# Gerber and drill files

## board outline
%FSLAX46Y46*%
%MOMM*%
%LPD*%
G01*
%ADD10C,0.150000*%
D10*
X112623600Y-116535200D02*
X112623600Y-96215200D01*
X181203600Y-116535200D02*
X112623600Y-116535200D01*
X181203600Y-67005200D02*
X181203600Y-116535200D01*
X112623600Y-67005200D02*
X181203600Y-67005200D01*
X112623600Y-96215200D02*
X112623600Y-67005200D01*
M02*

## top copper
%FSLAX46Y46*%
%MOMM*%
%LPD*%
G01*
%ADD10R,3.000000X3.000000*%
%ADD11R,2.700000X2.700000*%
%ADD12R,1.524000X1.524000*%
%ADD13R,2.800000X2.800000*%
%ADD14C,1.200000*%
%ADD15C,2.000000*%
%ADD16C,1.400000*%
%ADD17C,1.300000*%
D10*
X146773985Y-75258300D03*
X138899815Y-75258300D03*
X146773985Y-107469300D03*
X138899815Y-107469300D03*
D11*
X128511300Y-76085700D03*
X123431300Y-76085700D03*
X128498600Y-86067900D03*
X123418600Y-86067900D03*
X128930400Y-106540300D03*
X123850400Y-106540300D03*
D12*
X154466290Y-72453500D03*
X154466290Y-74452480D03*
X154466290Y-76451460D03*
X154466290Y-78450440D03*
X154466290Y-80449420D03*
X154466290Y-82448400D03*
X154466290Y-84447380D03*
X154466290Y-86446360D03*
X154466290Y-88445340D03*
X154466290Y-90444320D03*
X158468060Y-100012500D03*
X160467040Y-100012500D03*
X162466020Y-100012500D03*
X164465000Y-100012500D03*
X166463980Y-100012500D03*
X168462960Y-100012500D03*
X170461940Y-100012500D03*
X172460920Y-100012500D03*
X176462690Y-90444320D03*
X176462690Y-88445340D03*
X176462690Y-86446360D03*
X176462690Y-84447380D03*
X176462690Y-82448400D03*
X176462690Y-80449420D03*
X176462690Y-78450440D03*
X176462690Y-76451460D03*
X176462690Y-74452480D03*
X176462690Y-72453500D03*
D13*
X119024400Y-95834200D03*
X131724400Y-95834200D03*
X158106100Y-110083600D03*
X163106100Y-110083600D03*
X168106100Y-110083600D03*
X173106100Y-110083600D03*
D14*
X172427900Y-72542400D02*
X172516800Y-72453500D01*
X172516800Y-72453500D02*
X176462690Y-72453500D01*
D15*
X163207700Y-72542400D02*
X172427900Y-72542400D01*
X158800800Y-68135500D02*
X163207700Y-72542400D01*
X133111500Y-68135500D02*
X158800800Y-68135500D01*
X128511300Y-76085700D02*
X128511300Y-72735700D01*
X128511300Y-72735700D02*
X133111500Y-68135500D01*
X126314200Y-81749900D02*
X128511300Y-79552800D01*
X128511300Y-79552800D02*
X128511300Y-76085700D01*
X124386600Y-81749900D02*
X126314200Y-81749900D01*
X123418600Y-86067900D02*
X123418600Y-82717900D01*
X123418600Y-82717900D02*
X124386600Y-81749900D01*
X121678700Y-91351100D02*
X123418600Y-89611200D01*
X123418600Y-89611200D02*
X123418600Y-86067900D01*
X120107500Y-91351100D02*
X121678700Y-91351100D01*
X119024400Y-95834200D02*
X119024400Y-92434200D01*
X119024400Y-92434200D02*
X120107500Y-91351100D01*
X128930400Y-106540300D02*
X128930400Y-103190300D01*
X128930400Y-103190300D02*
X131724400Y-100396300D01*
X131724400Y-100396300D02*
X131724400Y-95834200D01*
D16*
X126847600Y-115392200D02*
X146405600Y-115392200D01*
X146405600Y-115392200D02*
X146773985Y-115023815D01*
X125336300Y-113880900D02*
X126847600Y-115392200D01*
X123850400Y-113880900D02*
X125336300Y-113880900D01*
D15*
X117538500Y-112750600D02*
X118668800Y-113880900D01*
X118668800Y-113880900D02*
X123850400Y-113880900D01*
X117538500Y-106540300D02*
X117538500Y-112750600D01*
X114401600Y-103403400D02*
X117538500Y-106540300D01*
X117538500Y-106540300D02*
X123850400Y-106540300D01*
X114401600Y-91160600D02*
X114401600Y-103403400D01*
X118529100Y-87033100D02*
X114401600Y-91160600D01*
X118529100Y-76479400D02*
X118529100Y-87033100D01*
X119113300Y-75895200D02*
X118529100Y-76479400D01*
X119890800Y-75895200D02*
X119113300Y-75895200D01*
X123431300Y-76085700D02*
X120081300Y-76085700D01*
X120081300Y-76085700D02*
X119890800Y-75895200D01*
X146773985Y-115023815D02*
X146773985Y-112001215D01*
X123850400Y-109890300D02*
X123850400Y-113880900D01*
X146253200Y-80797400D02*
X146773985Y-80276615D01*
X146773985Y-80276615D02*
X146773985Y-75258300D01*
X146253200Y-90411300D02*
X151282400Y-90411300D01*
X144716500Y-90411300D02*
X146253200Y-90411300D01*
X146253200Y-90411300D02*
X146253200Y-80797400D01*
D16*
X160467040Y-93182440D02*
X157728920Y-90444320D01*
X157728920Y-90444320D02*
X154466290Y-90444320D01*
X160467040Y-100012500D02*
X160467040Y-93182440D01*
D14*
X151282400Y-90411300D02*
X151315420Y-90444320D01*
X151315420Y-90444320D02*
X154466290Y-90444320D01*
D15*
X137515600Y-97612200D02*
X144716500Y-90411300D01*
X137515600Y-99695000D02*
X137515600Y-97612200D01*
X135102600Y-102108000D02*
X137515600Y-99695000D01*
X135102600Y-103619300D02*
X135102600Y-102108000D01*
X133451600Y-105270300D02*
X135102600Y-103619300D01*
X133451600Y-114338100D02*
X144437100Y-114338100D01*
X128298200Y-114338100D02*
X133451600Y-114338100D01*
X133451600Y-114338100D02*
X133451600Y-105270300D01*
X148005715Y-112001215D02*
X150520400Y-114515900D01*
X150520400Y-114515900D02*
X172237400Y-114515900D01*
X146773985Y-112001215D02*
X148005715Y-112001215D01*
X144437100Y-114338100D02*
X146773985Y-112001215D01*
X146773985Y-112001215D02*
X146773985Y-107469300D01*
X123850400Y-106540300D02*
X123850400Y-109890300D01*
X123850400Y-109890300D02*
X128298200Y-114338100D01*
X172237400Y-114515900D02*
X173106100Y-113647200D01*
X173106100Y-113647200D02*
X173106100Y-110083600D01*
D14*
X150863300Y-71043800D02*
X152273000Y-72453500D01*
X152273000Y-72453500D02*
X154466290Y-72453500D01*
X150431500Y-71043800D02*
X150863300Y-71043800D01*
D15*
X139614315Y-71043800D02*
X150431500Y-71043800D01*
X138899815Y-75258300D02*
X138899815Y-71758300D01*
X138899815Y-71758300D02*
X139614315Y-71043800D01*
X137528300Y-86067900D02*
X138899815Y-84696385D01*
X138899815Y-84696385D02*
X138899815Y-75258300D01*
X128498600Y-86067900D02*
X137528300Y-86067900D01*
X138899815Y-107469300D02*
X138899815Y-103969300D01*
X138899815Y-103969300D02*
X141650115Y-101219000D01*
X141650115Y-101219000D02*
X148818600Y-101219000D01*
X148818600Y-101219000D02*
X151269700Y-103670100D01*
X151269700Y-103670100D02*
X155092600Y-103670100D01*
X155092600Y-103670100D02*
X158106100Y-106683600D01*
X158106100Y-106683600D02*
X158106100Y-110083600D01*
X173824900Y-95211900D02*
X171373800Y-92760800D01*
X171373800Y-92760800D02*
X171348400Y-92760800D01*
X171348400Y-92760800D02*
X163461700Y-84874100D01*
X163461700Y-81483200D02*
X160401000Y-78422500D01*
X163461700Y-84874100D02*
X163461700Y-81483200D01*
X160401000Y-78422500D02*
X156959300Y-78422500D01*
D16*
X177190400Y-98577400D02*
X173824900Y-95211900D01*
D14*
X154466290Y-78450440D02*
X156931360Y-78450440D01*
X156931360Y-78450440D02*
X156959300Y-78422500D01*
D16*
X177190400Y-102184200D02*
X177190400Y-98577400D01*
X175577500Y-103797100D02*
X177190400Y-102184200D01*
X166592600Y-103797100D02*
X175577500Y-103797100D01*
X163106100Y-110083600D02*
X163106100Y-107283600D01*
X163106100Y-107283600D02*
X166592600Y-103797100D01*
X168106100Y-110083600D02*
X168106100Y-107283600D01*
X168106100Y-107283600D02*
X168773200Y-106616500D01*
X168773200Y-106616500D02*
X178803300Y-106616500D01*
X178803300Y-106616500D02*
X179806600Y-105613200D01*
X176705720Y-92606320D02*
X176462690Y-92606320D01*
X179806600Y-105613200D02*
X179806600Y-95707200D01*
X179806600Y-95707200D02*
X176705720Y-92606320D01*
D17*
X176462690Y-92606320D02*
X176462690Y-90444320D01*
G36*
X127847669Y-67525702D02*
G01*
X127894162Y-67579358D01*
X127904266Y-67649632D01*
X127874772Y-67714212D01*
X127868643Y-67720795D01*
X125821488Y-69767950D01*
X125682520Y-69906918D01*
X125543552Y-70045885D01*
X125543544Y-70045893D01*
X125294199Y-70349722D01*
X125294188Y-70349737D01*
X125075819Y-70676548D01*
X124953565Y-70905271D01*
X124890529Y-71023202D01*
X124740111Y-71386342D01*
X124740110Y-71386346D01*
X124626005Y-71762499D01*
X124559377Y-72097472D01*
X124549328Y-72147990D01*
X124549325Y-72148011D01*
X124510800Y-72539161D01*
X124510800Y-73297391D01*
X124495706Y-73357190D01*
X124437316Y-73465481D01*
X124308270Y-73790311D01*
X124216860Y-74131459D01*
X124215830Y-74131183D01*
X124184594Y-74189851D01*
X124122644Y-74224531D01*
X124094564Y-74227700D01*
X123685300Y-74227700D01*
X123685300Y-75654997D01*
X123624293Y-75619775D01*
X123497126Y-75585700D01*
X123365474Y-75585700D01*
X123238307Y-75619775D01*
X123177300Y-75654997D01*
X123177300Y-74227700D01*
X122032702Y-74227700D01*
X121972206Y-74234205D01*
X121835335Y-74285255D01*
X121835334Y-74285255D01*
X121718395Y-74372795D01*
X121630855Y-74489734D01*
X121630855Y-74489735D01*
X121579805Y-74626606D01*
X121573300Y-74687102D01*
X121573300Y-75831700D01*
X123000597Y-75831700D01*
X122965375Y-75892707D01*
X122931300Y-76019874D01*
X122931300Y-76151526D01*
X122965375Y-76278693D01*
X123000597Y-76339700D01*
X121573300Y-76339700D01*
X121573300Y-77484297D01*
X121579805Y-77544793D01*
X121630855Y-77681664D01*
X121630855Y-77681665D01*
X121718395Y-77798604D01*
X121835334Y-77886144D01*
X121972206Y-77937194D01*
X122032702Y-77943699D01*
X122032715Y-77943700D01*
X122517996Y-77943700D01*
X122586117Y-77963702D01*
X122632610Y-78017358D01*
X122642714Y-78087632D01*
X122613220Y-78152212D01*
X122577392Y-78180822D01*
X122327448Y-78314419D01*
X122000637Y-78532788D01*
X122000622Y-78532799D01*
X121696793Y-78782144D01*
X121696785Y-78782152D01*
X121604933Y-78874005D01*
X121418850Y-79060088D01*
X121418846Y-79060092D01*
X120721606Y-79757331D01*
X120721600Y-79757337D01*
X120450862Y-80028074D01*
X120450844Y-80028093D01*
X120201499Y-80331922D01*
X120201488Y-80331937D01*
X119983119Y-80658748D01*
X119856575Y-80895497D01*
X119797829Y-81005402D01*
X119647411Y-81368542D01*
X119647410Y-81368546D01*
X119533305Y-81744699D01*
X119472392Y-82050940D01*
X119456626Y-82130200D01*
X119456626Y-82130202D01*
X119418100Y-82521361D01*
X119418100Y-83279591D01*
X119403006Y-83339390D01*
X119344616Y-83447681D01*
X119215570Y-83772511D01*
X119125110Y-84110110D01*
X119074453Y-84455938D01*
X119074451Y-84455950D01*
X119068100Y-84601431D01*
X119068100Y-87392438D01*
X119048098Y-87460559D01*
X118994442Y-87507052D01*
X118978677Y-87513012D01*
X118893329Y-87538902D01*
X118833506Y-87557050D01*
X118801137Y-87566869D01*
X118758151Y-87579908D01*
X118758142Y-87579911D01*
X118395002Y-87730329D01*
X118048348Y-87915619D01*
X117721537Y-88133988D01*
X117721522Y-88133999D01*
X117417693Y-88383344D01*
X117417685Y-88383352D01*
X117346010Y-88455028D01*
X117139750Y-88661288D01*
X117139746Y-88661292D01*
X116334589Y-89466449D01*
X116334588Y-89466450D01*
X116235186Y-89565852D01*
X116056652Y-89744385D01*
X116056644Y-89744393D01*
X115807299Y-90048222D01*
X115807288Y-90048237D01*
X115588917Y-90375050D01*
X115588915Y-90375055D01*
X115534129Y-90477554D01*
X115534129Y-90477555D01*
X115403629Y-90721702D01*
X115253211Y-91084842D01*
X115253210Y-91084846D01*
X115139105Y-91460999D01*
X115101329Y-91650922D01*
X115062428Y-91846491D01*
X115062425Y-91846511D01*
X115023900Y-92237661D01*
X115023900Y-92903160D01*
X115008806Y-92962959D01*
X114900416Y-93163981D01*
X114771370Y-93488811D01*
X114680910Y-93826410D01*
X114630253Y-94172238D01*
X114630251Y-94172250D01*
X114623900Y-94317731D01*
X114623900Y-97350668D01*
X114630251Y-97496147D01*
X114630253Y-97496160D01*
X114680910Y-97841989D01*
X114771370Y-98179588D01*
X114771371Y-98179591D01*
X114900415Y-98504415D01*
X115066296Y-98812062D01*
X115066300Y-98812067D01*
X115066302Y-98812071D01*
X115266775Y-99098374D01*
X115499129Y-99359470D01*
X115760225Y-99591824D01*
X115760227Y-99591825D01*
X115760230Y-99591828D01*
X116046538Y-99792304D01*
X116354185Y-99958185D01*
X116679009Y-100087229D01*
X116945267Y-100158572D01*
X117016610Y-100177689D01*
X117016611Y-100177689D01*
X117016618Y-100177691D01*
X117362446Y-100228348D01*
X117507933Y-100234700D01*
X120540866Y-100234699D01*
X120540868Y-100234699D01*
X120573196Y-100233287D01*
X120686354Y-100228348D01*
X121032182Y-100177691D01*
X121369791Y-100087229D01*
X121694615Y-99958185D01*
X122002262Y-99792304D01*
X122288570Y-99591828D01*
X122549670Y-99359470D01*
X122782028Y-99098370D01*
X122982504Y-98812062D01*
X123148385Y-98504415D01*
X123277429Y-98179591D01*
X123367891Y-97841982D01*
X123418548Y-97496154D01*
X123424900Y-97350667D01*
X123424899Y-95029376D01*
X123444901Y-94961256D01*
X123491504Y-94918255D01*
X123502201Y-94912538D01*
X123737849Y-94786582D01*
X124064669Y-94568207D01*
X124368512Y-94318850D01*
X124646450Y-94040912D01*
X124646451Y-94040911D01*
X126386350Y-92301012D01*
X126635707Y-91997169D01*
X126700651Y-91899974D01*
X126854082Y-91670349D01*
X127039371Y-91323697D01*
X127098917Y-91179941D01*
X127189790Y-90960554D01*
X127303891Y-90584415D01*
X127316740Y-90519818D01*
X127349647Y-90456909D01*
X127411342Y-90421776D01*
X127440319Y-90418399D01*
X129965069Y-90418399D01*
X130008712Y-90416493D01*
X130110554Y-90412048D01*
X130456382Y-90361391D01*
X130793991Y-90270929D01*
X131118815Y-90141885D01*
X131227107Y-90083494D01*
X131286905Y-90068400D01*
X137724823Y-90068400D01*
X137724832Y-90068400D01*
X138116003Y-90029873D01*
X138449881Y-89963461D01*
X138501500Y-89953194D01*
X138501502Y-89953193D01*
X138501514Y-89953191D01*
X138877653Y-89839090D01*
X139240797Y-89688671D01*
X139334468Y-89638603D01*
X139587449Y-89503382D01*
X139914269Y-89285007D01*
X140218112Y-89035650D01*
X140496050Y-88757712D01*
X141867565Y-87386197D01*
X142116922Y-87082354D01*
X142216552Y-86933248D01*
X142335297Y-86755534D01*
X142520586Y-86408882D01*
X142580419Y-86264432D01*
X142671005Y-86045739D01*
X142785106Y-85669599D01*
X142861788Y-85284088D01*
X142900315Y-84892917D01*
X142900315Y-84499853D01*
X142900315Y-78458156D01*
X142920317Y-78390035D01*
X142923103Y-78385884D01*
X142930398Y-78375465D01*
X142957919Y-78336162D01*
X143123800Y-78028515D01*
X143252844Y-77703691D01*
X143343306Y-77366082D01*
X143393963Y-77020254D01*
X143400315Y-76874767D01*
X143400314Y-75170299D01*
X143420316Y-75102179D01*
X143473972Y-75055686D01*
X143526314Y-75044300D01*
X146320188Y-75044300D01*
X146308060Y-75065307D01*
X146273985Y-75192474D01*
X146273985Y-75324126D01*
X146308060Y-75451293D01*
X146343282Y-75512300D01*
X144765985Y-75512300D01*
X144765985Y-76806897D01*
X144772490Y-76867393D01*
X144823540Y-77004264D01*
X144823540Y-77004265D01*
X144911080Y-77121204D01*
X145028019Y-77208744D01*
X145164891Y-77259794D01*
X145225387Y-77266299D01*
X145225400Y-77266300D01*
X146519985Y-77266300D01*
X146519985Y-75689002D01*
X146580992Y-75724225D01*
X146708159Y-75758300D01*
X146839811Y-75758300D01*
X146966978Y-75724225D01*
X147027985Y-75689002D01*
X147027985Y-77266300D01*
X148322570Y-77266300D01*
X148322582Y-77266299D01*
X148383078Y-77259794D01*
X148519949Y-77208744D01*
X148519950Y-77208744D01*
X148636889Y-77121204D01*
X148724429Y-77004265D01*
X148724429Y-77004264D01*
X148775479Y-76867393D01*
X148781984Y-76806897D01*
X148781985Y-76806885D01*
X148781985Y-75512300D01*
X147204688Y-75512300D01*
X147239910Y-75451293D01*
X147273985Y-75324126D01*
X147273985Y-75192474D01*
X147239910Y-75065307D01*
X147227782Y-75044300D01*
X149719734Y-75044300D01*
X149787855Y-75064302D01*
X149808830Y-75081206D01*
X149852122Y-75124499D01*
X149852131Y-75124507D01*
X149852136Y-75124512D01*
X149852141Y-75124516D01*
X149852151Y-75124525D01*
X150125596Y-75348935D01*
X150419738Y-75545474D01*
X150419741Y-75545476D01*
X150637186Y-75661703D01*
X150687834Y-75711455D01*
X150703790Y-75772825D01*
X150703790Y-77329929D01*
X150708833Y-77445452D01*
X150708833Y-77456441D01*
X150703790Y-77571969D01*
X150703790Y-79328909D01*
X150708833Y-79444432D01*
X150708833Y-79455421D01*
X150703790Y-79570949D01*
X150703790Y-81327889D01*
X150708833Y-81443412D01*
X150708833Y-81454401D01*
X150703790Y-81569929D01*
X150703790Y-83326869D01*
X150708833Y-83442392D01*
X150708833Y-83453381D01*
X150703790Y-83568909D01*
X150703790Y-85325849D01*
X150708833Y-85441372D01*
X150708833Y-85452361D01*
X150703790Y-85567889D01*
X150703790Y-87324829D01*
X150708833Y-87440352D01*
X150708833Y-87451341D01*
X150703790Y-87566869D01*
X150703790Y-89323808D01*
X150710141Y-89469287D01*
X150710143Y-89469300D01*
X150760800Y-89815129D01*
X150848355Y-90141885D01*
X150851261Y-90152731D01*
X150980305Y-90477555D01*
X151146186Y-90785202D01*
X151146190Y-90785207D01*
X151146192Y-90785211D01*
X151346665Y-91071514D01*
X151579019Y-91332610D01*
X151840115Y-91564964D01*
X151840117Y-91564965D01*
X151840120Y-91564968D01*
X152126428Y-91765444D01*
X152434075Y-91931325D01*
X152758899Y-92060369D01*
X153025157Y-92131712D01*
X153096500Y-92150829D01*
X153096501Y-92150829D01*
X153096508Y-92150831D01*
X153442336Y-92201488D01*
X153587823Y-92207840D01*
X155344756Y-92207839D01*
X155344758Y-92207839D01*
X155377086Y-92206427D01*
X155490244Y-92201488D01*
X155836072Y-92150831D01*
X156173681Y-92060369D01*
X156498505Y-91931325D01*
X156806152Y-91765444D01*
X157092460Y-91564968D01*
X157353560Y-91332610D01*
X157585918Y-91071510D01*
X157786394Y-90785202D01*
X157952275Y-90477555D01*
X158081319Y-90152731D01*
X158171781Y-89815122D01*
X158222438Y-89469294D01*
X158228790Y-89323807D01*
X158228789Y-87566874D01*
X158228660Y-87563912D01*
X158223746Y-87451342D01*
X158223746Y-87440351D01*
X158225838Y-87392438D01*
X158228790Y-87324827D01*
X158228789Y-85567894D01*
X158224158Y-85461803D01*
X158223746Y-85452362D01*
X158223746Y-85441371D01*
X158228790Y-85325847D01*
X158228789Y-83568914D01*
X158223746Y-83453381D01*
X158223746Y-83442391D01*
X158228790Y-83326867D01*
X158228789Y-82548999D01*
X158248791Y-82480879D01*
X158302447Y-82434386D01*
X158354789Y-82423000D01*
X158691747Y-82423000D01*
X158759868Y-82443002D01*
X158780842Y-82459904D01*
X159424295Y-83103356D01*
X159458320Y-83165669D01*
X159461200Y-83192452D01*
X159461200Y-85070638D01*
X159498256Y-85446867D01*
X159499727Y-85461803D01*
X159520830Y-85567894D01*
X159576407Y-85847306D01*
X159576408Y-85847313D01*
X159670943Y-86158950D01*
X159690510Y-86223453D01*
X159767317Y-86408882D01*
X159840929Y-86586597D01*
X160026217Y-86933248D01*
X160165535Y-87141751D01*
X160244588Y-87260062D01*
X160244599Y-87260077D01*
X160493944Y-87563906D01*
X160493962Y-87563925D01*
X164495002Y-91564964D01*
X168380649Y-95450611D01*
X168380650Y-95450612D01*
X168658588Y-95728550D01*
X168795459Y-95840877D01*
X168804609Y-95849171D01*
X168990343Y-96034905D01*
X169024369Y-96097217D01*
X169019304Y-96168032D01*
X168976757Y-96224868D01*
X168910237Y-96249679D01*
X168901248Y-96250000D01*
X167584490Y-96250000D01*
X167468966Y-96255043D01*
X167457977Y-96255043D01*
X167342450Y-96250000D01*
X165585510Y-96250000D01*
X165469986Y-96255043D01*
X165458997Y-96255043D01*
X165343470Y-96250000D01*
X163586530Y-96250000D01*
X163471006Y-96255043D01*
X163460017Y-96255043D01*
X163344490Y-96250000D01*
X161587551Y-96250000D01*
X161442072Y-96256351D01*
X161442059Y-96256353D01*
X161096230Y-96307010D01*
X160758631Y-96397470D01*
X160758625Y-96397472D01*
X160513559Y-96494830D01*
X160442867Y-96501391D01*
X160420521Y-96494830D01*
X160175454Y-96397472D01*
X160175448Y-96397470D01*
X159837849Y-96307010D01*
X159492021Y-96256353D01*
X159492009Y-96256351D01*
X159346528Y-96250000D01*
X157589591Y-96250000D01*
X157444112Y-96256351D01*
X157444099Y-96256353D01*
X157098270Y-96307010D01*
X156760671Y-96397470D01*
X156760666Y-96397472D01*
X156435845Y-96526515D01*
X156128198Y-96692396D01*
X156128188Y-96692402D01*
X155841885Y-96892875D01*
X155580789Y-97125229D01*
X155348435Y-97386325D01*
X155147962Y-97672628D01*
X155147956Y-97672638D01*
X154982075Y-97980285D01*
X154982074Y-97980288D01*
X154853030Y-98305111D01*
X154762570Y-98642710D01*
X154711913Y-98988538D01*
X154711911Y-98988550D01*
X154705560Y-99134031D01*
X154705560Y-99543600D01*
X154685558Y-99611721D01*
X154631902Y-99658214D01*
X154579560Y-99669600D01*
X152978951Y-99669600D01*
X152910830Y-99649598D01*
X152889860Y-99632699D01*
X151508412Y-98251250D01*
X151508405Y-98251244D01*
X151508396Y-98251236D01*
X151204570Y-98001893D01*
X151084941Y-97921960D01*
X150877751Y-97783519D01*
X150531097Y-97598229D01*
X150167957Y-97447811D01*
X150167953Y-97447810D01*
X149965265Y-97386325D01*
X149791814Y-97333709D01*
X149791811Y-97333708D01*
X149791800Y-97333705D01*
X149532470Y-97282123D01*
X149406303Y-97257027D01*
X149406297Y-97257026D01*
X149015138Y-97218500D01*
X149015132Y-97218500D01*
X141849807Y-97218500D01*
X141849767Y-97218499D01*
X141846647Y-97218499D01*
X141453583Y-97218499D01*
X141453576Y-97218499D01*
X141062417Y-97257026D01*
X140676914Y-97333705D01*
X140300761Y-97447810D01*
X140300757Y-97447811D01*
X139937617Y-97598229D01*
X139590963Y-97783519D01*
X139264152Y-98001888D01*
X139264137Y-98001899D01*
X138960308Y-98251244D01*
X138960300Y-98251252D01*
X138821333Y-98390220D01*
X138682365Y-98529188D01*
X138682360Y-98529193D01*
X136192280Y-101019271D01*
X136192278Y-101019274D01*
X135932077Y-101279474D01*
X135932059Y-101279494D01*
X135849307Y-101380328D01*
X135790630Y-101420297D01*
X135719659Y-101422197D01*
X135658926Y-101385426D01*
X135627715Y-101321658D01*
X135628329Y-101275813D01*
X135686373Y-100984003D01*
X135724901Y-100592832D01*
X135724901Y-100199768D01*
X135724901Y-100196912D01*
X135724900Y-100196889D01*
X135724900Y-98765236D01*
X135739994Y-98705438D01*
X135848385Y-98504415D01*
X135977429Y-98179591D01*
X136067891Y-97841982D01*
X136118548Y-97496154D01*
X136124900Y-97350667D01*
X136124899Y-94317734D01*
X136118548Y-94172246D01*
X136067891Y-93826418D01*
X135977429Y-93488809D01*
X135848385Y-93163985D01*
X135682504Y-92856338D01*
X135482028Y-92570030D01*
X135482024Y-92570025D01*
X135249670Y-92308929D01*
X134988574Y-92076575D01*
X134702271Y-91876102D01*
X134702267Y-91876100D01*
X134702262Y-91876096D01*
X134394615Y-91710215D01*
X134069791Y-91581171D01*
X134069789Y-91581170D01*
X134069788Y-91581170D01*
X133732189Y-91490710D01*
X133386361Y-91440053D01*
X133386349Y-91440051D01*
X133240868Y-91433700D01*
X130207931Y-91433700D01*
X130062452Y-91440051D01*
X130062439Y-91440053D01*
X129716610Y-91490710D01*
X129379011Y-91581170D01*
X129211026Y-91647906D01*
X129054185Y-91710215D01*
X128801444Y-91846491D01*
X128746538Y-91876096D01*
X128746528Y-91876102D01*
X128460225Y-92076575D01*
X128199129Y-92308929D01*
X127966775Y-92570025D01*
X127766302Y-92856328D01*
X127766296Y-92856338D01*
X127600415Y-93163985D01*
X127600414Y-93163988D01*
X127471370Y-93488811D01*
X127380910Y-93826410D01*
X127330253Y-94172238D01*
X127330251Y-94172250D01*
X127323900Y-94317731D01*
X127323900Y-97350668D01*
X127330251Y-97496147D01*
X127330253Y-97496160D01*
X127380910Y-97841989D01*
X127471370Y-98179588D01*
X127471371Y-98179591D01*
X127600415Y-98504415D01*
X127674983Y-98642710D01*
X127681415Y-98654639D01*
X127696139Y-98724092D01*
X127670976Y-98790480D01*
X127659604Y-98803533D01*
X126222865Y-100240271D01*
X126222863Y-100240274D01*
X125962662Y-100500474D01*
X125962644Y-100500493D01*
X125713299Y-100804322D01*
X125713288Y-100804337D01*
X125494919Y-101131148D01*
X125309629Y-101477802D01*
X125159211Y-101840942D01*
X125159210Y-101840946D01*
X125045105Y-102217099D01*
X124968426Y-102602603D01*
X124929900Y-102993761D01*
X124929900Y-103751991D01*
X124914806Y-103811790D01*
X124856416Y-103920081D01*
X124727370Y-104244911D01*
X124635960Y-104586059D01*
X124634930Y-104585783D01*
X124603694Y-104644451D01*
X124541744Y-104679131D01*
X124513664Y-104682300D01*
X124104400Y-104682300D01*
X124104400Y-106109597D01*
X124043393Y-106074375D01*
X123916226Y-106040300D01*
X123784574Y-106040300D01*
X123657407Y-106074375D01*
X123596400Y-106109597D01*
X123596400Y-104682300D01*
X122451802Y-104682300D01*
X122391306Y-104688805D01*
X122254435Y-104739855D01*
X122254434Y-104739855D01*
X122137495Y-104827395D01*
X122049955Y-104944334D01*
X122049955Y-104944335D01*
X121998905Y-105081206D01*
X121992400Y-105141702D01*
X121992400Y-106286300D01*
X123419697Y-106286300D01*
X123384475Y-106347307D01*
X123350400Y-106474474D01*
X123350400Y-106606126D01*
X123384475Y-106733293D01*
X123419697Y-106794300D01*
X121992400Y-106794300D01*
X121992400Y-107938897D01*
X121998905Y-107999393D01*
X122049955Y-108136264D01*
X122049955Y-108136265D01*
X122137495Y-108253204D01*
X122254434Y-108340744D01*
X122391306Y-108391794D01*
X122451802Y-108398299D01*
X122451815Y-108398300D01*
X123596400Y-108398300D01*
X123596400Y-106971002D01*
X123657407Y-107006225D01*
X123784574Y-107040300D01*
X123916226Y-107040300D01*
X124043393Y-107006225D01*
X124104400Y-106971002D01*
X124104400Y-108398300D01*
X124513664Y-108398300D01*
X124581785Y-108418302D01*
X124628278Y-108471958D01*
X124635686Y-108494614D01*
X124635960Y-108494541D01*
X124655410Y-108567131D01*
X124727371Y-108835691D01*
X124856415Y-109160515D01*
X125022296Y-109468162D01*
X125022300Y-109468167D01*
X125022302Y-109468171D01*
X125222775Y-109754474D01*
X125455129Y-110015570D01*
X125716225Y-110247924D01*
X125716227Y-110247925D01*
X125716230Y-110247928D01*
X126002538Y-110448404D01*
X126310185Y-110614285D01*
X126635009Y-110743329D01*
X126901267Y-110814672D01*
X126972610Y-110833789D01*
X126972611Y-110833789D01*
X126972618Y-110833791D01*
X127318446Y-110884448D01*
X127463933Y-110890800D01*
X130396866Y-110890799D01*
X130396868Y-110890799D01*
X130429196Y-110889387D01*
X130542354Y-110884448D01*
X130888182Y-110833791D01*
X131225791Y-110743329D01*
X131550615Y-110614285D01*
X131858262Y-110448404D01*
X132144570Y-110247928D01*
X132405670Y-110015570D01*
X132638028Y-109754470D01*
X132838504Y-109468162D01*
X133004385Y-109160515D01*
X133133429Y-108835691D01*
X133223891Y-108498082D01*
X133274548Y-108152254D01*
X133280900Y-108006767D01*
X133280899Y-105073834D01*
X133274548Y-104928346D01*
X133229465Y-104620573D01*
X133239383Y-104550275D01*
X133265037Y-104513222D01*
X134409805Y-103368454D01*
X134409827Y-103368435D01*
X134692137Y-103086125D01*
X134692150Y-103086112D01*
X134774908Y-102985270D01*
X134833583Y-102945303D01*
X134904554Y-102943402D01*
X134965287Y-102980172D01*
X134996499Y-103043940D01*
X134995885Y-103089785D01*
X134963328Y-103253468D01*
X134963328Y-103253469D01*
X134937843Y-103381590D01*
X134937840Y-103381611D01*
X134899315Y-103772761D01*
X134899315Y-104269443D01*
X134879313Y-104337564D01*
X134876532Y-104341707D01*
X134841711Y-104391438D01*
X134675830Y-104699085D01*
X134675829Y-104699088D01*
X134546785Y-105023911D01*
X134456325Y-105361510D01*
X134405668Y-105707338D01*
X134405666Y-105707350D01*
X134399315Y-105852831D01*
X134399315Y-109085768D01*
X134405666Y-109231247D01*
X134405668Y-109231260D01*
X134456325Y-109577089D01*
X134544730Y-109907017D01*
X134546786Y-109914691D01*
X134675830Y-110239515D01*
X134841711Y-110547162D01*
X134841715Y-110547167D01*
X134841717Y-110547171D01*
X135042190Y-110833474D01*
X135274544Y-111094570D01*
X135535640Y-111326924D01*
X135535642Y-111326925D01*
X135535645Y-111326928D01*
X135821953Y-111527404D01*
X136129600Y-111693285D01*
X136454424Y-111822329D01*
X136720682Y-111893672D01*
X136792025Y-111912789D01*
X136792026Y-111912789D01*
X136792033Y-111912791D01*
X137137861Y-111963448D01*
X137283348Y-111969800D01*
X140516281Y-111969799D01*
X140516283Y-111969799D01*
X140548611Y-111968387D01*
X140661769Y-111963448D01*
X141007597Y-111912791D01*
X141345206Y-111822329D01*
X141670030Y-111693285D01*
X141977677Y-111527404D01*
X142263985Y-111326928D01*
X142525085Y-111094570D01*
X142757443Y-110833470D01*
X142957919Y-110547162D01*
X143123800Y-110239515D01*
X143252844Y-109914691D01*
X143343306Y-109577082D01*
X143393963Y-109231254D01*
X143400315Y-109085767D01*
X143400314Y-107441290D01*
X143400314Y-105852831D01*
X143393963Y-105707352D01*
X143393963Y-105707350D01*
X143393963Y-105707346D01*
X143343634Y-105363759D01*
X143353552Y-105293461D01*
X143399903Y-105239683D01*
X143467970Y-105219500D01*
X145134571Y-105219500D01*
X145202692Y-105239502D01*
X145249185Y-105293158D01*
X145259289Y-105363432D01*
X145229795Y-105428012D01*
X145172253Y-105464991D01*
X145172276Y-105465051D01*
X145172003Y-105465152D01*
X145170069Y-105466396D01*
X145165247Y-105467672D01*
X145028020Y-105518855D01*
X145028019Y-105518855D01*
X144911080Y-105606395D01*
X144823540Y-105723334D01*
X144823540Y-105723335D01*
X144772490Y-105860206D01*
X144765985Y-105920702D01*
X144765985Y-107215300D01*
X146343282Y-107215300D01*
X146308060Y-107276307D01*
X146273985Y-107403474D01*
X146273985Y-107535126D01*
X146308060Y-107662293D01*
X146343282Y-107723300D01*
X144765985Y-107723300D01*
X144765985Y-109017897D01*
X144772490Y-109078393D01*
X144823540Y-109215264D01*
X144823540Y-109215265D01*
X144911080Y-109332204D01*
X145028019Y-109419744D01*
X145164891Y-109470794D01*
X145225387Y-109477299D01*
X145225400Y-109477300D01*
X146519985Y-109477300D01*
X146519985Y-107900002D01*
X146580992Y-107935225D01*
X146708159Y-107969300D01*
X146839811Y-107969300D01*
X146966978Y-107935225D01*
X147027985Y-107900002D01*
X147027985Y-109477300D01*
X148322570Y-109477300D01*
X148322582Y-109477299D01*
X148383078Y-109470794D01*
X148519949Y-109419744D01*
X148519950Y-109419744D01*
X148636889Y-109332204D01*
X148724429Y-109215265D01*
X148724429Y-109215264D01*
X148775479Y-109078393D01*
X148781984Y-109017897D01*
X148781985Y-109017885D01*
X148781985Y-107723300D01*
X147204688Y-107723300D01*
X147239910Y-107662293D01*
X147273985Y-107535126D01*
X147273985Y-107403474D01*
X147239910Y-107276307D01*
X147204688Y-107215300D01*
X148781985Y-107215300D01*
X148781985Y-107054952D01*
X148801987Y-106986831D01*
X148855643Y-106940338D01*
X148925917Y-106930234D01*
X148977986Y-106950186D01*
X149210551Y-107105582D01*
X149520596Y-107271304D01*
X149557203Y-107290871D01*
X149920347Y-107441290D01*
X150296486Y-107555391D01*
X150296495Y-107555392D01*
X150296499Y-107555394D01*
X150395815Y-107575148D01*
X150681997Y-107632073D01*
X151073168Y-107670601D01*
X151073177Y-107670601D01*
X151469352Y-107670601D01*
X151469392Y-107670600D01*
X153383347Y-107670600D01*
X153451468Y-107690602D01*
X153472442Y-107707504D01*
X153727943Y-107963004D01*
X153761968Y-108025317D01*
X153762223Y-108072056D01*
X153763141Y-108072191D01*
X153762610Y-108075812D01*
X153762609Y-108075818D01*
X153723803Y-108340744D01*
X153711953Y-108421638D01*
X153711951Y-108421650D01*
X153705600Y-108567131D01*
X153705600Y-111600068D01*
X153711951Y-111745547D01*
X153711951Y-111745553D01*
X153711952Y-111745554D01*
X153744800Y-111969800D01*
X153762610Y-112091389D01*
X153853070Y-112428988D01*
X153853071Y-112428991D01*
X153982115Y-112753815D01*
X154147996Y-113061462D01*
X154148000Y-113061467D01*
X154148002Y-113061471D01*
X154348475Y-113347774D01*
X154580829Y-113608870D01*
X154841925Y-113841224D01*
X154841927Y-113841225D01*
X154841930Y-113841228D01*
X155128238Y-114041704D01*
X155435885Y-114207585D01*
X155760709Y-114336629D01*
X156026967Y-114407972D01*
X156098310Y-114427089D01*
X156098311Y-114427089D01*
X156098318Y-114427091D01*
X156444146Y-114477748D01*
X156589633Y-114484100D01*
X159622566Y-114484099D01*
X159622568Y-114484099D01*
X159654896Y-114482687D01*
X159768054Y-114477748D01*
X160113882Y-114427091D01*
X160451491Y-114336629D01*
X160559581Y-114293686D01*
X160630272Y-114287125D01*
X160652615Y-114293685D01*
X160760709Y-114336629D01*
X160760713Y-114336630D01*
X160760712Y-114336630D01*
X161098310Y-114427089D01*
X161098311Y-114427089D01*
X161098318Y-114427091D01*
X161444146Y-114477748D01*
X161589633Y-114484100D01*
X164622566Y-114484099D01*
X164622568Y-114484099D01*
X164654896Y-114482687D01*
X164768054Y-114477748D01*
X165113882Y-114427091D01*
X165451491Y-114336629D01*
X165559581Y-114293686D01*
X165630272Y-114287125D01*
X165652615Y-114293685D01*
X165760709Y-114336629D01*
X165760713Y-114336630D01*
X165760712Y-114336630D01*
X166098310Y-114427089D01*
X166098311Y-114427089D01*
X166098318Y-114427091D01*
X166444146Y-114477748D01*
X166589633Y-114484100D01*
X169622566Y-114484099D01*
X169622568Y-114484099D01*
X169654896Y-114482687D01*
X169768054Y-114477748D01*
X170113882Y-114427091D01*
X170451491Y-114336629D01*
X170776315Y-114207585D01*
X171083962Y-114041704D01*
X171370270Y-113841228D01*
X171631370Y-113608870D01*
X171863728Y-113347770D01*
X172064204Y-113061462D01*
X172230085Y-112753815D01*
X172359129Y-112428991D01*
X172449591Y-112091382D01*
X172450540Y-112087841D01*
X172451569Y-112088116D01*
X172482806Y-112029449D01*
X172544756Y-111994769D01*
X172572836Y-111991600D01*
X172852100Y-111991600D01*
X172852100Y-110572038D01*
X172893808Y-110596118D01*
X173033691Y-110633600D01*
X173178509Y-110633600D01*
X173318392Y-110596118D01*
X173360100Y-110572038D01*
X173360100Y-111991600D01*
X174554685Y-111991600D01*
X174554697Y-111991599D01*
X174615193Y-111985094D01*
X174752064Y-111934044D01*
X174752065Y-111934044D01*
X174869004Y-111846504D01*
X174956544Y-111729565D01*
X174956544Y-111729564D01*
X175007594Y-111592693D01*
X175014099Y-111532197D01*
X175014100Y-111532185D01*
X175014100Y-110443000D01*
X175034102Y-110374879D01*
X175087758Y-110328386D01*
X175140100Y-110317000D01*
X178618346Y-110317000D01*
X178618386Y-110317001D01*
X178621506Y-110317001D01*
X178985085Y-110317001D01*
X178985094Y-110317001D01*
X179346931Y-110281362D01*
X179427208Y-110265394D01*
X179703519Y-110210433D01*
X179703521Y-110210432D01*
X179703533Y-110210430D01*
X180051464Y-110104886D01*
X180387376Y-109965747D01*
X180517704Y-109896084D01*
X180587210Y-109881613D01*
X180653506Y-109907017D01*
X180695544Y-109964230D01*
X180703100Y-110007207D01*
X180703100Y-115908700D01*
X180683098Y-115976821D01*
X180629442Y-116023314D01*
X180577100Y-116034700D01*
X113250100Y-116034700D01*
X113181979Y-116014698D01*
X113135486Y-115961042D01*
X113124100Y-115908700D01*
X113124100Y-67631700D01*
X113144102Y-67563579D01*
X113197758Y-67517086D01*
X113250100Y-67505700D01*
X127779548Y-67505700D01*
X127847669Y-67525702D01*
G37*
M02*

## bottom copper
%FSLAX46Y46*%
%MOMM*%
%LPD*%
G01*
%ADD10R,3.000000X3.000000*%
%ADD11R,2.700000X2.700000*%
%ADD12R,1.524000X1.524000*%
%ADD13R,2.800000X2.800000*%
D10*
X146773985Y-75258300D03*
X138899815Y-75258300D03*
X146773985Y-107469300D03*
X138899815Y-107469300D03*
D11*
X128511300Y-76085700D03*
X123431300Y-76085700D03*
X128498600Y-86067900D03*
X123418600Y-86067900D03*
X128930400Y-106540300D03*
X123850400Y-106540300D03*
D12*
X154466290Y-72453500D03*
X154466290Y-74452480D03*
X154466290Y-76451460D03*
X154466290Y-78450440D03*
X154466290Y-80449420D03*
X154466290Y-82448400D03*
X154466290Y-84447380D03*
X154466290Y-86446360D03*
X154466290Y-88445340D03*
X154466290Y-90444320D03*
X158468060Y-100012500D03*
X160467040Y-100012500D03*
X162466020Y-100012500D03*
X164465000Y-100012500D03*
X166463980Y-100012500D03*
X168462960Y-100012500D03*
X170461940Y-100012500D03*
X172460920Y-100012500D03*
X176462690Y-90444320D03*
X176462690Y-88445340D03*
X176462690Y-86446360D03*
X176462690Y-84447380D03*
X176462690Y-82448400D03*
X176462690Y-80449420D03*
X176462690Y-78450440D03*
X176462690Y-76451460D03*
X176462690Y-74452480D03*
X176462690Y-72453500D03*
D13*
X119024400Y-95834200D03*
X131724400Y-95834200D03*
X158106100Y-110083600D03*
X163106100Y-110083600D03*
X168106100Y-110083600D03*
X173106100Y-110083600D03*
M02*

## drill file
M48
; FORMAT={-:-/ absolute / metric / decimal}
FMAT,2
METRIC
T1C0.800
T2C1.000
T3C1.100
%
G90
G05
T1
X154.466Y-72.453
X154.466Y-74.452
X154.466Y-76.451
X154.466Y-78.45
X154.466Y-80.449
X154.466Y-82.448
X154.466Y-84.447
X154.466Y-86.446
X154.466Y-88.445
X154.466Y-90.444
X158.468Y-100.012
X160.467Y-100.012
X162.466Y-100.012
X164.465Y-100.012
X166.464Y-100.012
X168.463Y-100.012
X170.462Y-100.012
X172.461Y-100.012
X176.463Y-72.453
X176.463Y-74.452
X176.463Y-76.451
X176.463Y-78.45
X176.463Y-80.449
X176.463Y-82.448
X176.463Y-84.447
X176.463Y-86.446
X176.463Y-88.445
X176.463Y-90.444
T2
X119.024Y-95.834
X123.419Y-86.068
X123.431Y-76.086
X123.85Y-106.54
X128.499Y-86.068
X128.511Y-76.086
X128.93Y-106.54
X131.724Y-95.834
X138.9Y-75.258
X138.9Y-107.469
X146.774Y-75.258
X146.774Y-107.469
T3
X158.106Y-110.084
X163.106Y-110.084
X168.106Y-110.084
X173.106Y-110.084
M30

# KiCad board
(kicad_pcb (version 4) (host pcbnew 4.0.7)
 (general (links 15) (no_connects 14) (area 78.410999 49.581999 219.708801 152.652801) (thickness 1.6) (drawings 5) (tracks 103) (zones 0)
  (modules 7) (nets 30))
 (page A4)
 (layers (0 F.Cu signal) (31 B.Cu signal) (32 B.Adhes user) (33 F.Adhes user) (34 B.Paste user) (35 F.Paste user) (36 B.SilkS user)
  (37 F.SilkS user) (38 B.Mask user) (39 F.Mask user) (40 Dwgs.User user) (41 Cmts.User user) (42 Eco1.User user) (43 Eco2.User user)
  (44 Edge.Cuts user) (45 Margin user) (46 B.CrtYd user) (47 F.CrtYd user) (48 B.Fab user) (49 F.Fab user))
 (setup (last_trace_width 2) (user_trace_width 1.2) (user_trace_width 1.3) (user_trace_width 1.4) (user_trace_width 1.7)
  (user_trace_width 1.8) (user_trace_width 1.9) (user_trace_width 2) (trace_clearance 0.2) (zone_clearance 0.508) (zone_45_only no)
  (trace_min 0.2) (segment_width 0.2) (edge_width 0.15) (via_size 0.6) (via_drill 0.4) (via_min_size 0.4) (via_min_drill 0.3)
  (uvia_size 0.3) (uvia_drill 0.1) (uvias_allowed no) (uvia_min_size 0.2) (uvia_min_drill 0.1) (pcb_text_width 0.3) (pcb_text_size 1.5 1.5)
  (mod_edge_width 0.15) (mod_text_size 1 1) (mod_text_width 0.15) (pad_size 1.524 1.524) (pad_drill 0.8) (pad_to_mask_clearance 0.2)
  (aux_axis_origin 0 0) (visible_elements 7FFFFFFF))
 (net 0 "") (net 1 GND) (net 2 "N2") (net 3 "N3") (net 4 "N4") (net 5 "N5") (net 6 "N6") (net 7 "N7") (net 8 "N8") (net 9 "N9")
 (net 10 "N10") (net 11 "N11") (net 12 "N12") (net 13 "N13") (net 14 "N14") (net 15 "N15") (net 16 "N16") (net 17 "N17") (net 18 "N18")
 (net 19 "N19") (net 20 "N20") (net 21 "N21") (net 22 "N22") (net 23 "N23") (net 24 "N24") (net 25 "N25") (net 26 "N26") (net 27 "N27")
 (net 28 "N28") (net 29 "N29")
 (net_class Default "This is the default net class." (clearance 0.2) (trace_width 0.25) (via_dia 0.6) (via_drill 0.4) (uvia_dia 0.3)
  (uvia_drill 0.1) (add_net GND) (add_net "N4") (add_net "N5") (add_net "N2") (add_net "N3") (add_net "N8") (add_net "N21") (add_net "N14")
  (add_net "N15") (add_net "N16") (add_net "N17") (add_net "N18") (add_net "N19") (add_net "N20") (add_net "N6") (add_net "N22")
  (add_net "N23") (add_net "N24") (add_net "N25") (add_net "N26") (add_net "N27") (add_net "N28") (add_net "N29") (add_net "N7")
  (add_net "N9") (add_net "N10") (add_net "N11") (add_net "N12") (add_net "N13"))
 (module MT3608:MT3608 (layer F.Cu) (at 142.8369 91.3638 270)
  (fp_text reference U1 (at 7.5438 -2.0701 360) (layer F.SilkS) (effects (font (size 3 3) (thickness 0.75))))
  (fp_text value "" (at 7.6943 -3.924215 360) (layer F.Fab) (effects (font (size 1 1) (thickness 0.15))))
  (pad 2 thru_hole rect (at -16.1055 -3.937085 270) (size 3 3) (drill 1) (layers *.Cu *.Mask) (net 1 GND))
  (pad 1 thru_hole rect (at -16.1055 3.937085 270) (size 3 3) (drill 1) (layers *.Cu *.Mask) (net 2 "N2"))
  (pad 4 thru_hole rect (at 16.1055 -3.937085 270) (size 3 3) (drill 1) (layers *.Cu *.Mask) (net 1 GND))
  (pad 3 thru_hole rect (at 16.1055 3.937085 270) (size 3 3) (drill 1) (layers *.Cu *.Mask) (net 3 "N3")))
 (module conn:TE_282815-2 (layer F.Cu) (at 125.9713 76.0857 180)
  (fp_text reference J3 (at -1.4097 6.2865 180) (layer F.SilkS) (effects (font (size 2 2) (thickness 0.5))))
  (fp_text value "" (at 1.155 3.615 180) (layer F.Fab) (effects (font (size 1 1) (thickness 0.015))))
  (pad 1 thru_hole rect (at -2.54 0 180) (size 2.7 2.7) (drill 1) (layers *.Cu *.Mask) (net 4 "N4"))
  (pad 2 thru_hole rect (at 2.54 0 180) (size 2.7 2.7) (drill 1) (layers *.Cu *.Mask) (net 1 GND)))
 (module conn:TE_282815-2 (layer F.Cu) (at 125.9586 86.0679 180)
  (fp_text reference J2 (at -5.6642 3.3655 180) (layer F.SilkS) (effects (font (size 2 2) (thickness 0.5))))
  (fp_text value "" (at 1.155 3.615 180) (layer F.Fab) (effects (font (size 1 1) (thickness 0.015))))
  (pad 1 thru_hole rect (at -2.54 0 180) (size 2.7 2.7) (drill 1) (layers *.Cu *.Mask) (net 2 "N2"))
  (pad 2 thru_hole rect (at 2.54 0 180) (size 2.7 2.7) (drill 1) (layers *.Cu *.Mask) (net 4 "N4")))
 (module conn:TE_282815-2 (layer F.Cu) (at 126.3904 106.5403 180)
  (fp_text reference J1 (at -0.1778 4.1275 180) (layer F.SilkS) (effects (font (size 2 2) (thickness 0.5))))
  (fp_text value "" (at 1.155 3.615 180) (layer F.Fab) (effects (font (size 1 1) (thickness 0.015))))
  (pad 1 thru_hole rect (at -2.54 0 180) (size 2.7 2.7) (drill 1) (layers *.Cu *.Mask) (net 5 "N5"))
  (pad 2 thru_hole rect (at 2.54 0 180) (size 2.7 2.7) (drill 1) (layers *.Cu *.Mask) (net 1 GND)))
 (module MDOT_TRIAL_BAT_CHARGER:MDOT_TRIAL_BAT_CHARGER (layer F.Cu) (at 165.46449 85.44687)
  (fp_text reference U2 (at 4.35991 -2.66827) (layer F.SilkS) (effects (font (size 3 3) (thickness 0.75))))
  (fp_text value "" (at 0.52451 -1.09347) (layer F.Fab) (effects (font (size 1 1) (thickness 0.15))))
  (pad 1 thru_hole rect (at -10.9982 -12.99337) (size 1.524 1.524) (drill 0.8) (layers *.Cu *.Mask) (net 2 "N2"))
  (pad 2 thru_hole rect (at -10.9982 -10.99439) (size 1.524 1.524) (drill 0.8) (layers *.Cu *.Mask) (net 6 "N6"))
  (pad 3 thru_hole rect (at -10.9982 -8.99541) (size 1.524 1.524) (drill 0.8) (layers *.Cu *.Mask) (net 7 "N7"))
  (pad 4 thru_hole rect (at -10.9982 -6.99643) (size 1.524 1.524) (drill 0.8) (layers *.Cu *.Mask) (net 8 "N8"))
  (pad 5 thru_hole rect (at -10.9982 -4.99745) (size 1.524 1.524) (drill 0.8) (layers *.Cu *.Mask) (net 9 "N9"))
  (pad 6 thru_hole rect (at -10.9982 -2.99847) (size 1.524 1.524) (drill 0.8) (layers *.Cu *.Mask) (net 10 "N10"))
  (pad 7 thru_hole rect (at -10.9982 -0.99949) (size 1.524 1.524) (drill 0.8) (layers *.Cu *.Mask) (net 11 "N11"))
  (pad 8 thru_hole rect (at -10.9982 0.99949) (size 1.524 1.524) (drill 0.8) (layers *.Cu *.Mask) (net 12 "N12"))
  (pad 9 thru_hole rect (at -10.9982 2.99847) (size 1.524 1.524) (drill 0.8) (layers *.Cu *.Mask) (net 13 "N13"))
  (pad 10 thru_hole rect (at -10.9982 4.99745) (size 1.524 1.524) (drill 0.8) (layers *.Cu *.Mask) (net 1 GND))
  (pad 11 thru_hole rect (at -6.99643 14.56563) (size 1.524 1.524) (drill 0.8) (layers *.Cu *.Mask) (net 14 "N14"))
  (pad 12 thru_hole rect (at -4.99745 14.56563) (size 1.524 1.524) (drill 0.8) (layers *.Cu *.Mask) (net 1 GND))
  (pad 13 thru_hole rect (at -2.99847 14.56563) (size 1.524 1.524) (drill 0.8) (layers *.Cu *.Mask) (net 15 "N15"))
  (pad 14 thru_hole rect (at -0.99949 14.56563) (size 1.524 1.524) (drill 0.8) (layers *.Cu *.Mask) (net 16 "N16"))
  (pad 15 thru_hole rect (at 0.99949 14.56563) (size 1.524 1.524) (drill 0.8) (layers *.Cu *.Mask) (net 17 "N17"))
  (pad 16 thru_hole rect (at 2.99847 14.56563) (size 1.524 1.524) (drill 0.8) (layers *.Cu *.Mask) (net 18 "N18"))
  (pad 17 thru_hole rect (at 4.99745 14.56563) (size 1.524 1.524) (drill 0.8) (layers *.Cu *.Mask) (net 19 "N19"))
  (pad 18 thru_hole rect (at 6.99643 14.56563) (size 1.524 1.524) (drill 0.8) (layers *.Cu *.Mask) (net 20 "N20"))
  (pad 19 thru_hole rect (at 10.9982 4.99745) (size 1.524 1.524) (drill 0.8) (layers *.Cu *.Mask) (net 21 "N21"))
  (pad 20 thru_hole rect (at 10.9982 2.99847) (size 1.524 1.524) (drill 0.8) (layers *.Cu *.Mask) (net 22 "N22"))
  (pad 21 thru_hole rect (at 10.9982 0.99949) (size 1.524 1.524) (drill 0.8) (layers *.Cu *.Mask) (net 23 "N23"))
  (pad 22 thru_hole rect (at 10.9982 -0.99949) (size 1.524 1.524) (drill 0.8) (layers *.Cu *.Mask) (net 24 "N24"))
  (pad 23 thru_hole rect (at 10.9982 -2.99847) (size 1.524 1.524) (drill 0.8) (layers *.Cu *.Mask) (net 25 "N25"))
  (pad 24 thru_hole rect (at 10.9982 -4.99745) (size 1.524 1.524) (drill 0.8) (layers *.Cu *.Mask) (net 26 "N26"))
  (pad 25 thru_hole rect (at 10.9982 -6.99643) (size 1.524 1.524) (drill 0.8) (layers *.Cu *.Mask) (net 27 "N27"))
  (pad 26 thru_hole rect (at 10.9982 -8.99541) (size 1.524 1.524) (drill 0.8) (layers *.Cu *.Mask) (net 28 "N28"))
  (pad 27 thru_hole rect (at 10.9982 -10.99439) (size 1.524 1.524) (drill 0.8) (layers *.Cu *.Mask) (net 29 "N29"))
  (pad 28 thru_hole rect (at 10.9982 -12.99337) (size 1.524 1.524) (drill 0.8) (layers *.Cu *.Mask) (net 4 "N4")))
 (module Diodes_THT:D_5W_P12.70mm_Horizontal (layer F.Cu) (at 119.0244 95.8342)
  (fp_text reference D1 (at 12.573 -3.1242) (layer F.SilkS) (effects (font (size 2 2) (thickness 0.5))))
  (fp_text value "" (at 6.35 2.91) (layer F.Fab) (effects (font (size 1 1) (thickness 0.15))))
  (pad 1 thru_hole rect (at 0 0) (size 2.8 2.8) (drill 1) (layers *.Cu *.Mask) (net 4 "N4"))
  (pad 2 thru_hole rect (at 12.7 0) (size 2.8 2.8) (drill 1) (layers *.Cu *.Mask) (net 5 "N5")))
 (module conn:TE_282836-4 (layer F.Cu) (at 165.6061 110.0836)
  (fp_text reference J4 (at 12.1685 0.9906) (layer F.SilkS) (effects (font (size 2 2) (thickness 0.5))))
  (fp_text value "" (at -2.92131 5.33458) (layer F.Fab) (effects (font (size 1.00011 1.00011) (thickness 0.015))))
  (pad 1 thru_hole rect (at -7.5 0) (size 2.8 2.8) (drill 1.1) (layers *.Cu *.Mask) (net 3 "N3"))
  (pad 2 thru_hole rect (at -2.5 0) (size 2.8 2.8) (drill 1.1) (layers *.Cu *.Mask) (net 8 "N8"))
  (pad 3 thru_hole rect (at 2.5 0) (size 2.8 2.8) (drill 1.1) (layers *.Cu *.Mask) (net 21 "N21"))
  (pad 4 thru_hole rect (at 7.5 0) (size 2.8 2.8) (drill 1.1) (layers *.Cu *.Mask) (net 1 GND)))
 (gr_line (start 112.6236 116.5352) (end 112.6236 96.2152) (layer Edge.Cuts) (width 0.15))
 (gr_line (start 181.2036 116.5352) (end 112.6236 116.5352) (layer Edge.Cuts) (width 0.15))
 (gr_line (start 181.2036 67.0052) (end 181.2036 116.5352) (layer Edge.Cuts) (width 0.15))
 (gr_line (start 112.6236 67.0052) (end 181.2036 67.0052) (layer Edge.Cuts) (width 0.15))
 (gr_line (start 112.6236 96.2152) (end 112.6236 67.0052) (layer Edge.Cuts) (width 0.15))
 (segment (start 172.4279 72.5424) (end 172.5168 72.4535) (width 1.2) (layer F.Cu) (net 4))
 (segment (start 172.5168 72.4535) (end 176.46269 72.4535) (width 1.2) (layer F.Cu) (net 4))
 (segment (start 163.2077 72.5424) (end 172.4279 72.5424) (width 2) (layer F.Cu) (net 4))
 (segment (start 158.8008 68.1355) (end 163.2077 72.5424) (width 2) (layer F.Cu) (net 4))
 (segment (start 133.1115 68.1355) (end 158.8008 68.1355) (width 2) (layer F.Cu) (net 4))
 (segment (start 128.5113 76.0857) (end 128.5113 72.7357) (width 2) (layer F.Cu) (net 4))
 (segment (start 128.5113 72.7357) (end 133.1115 68.1355) (width 2) (layer F.Cu) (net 4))
 (segment (start 126.3142 81.7499) (end 128.5113 79.5528) (width 2) (layer F.Cu) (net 4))
 (segment (start 128.5113 79.5528) (end 128.5113 76.0857) (width 2) (layer F.Cu) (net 4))
 (segment (start 124.3866 81.7499) (end 126.3142 81.7499) (width 2) (layer F.Cu) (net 4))
 (segment (start 123.4186 86.0679) (end 123.4186 82.7179) (width 2) (layer F.Cu) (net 4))
 (segment (start 123.4186 82.7179) (end 124.3866 81.7499) (width 2) (layer F.Cu) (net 4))
 (segment (start 121.6787 91.3511) (end 123.4186 89.6112) (width 2) (layer F.Cu) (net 4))
 (segment (start 123.4186 89.6112) (end 123.4186 86.0679) (width 2) (layer F.Cu) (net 4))
 (segment (start 120.1075 91.3511) (end 121.6787 91.3511) (width 2) (layer F.Cu) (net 4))
 (segment (start 119.0244 95.8342) (end 119.0244 92.4342) (width 2) (layer F.Cu) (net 4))
 (segment (start 119.0244 92.4342) (end 120.1075 91.3511) (width 2) (layer F.Cu) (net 4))
 (segment (start 128.9304 106.5403) (end 128.9304 103.1903) (width 2) (layer F.Cu) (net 5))
 (segment (start 128.9304 103.1903) (end 131.7244 100.3963) (width 2) (layer F.Cu) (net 5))
 (segment (start 131.7244 100.3963) (end 131.7244 95.8342) (width 2) (layer F.Cu) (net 5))
 (segment (start 126.8476 115.3922) (end 146.4056 115.3922) (width 1.4) (layer F.Cu) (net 1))
 (segment (start 146.4056 115.3922) (end 146.773985 115.023815) (width 1.4) (layer F.Cu) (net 1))
 (segment (start 125.3363 113.8809) (end 126.8476 115.3922) (width 1.4) (layer F.Cu) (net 1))
 (segment (start 123.8504 113.8809) (end 125.3363 113.8809) (width 1.4) (layer F.Cu) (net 1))
 (segment (start 117.5385 112.7506) (end 118.6688 113.8809) (width 2) (layer F.Cu) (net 1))
 (segment (start 118.6688 113.8809) (end 123.8504 113.8809) (width 2) (layer F.Cu) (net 1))
 (segment (start 117.5385 106.5403) (end 117.5385 112.7506) (width 2) (layer F.Cu) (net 1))
 (segment (start 114.4016 103.4034) (end 117.5385 106.5403) (width 2) (layer F.Cu) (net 1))
 (segment (start 117.5385 106.5403) (end 123.8504 106.5403) (width 2) (layer F.Cu) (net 1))
 (segment (start 114.4016 91.1606) (end 114.4016 103.4034) (width 2) (layer F.Cu) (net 1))
 (segment (start 118.5291 87.0331) (end 114.4016 91.1606) (width 2) (layer F.Cu) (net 1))
 (segment (start 118.5291 76.4794) (end 118.5291 87.0331) (width 2) (layer F.Cu) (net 1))
 (segment (start 119.1133 75.8952) (end 118.5291 76.4794) (width 2) (layer F.Cu) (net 1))
 (segment (start 119.8908 75.8952) (end 119.1133 75.8952) (width 2) (layer F.Cu) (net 1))
 (segment (start 123.4313 76.0857) (end 120.0813 76.0857) (width 2) (layer F.Cu) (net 1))
 (segment (start 120.0813 76.0857) (end 119.8908 75.8952) (width 2) (layer F.Cu) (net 1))
 (segment (start 146.773985 115.023815) (end 146.773985 112.001215) (width 2) (layer F.Cu) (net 1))
 (segment (start 123.8504 109.8903) (end 123.8504 113.8809) (width 2) (layer F.Cu) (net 1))
 (segment (start 146.2532 80.7974) (end 146.773985 80.276615) (width 2) (layer F.Cu) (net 1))
 (segment (start 146.773985 80.276615) (end 146.773985 75.2583) (width 2) (layer F.Cu) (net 1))
 (segment (start 146.2532 90.4113) (end 151.2824 90.4113) (width 2) (layer F.Cu) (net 1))
 (segment (start 144.7165 90.4113) (end 146.2532 90.4113) (width 2) (layer F.Cu) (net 1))
 (segment (start 146.2532 90.4113) (end 146.2532 80.7974) (width 2) (layer F.Cu) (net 1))
 (segment (start 160.46704 93.18244) (end 157.72892 90.44432) (width 1.4) (layer F.Cu) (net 1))
 (segment (start 157.72892 90.44432) (end 154.46629 90.44432) (width 1.4) (layer F.Cu) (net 1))
 (segment (start 160.46704 100.0125) (end 160.46704 93.18244) (width 1.4) (layer F.Cu) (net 1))
 (segment (start 151.2824 90.4113) (end 151.31542 90.44432) (width 1.2) (layer F.Cu) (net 1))
 (segment (start 151.31542 90.44432) (end 154.46629 90.44432) (width 1.2) (layer F.Cu) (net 1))
 (segment (start 137.5156 97.6122) (end 144.7165 90.4113) (width 2) (layer F.Cu) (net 1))
 (segment (start 137.5156 99.695) (end 137.5156 97.6122) (width 2) (layer F.Cu) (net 1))
 (segment (start 135.1026 102.108) (end 137.5156 99.695) (width 2) (layer F.Cu) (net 1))
 (segment (start 135.1026 103.6193) (end 135.1026 102.108) (width 2) (layer F.Cu) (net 1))
 (segment (start 133.4516 105.2703) (end 135.1026 103.6193) (width 2) (layer F.Cu) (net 1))
 (segment (start 133.4516 114.3381) (end 144.4371 114.3381) (width 2) (layer F.Cu) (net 1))
 (segment (start 128.2982 114.3381) (end 133.4516 114.3381) (width 2) (layer F.Cu) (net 1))
 (segment (start 133.4516 114.3381) (end 133.4516 105.2703) (width 2) (layer F.Cu) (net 1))
 (segment (start 148.005715 112.001215) (end 150.5204 114.5159) (width 2) (layer F.Cu) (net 1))
 (segment (start 150.5204 114.5159) (end 172.2374 114.5159) (width 2) (layer F.Cu) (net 1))
 (segment (start 146.773985 112.001215) (end 148.005715 112.001215) (width 2) (layer F.Cu) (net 1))
 (segment (start 144.4371 114.3381) (end 146.773985 112.001215) (width 2) (layer F.Cu) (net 1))
 (segment (start 146.773985 112.001215) (end 146.773985 107.4693) (width 2) (layer F.Cu) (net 1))
 (segment (start 123.8504 106.5403) (end 123.8504 109.8903) (width 2) (layer F.Cu) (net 1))
 (segment (start 123.8504 109.8903) (end 128.2982 114.3381) (width 2) (layer F.Cu) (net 1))
 (segment (start 172.2374 114.5159) (end 173.1061 113.6472) (width 2) (layer F.Cu) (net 1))
 (segment (start 173.1061 113.6472) (end 173.1061 110.0836) (width 2) (layer F.Cu) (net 1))
 (segment (start 150.8633 71.0438) (end 152.273 72.4535) (width 1.2) (layer F.Cu) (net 2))
 (segment (start 152.273 72.4535) (end 154.46629 72.4535) (width 1.2) (layer F.Cu) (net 2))
 (segment (start 150.4315 71.0438) (end 150.8633 71.0438) (width 1.2) (layer F.Cu) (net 2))
 (segment (start 139.614315 71.0438) (end 150.4315 71.0438) (width 2) (layer F.Cu) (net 2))
 (segment (start 138.899815 75.2583) (end 138.899815 71.7583) (width 2) (layer F.Cu) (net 2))
 (segment (start 138.899815 71.7583) (end 139.614315 71.0438) (width 2) (layer F.Cu) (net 2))
 (segment (start 137.5283 86.0679) (end 138.899815 84.696385) (width 2) (layer F.Cu) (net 2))
 (segment (start 138.899815 84.696385) (end 138.899815 75.2583) (width 2) (layer F.Cu) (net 2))
 (segment (start 128.4986 86.0679) (end 137.5283 86.0679) (width 2) (layer F.Cu) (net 2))
 (segment (start 138.899815 107.4693) (end 138.899815 103.9693) (width 2) (layer F.Cu) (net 3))
 (segment (start 138.899815 103.9693) (end 141.650115 101.219) (width 2) (layer F.Cu) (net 3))
 (segment (start 141.650115 101.219) (end 148.8186 101.219) (width 2) (layer F.Cu) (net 3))
 (segment (start 148.8186 101.219) (end 151.2697 103.6701) (width 2) (layer F.Cu) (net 3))
 (segment (start 151.2697 103.6701) (end 155.0926 103.6701) (width 2) (layer F.Cu) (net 3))
 (segment (start 155.0926 103.6701) (end 158.1061 106.6836) (width 2) (layer F.Cu) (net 3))
 (segment (start 158.1061 106.6836) (end 158.1061 110.0836) (width 2) (layer F.Cu) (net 3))
 (segment (start 173.8249 95.2119) (end 171.3738 92.7608) (width 2) (layer F.Cu) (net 8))
 (segment (start 171.3738 92.7608) (end 171.3484 92.7608) (width 2) (layer F.Cu) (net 8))
 (segment (start 171.3484 92.7608) (end 163.4617 84.8741) (width 2) (layer F.Cu) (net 8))
 (segment (start 163.4617 81.4832) (end 160.401 78.4225) (width 2) (layer F.Cu) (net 8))
 (segment (start 163.4617 84.8741) (end 163.4617 81.4832) (width 2) (layer F.Cu) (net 8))
 (segment (start 160.401 78.4225) (end 156.9593 78.4225) (width 2) (layer F.Cu) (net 8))
 (segment (start 177.1904 98.5774) (end 173.8249 95.2119) (width 1.4) (layer F.Cu) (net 8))
 (segment (start 154.46629 78.45044) (end 156.93136 78.45044) (width 1.2) (layer F.Cu) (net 8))
 (segment (start 156.93136 78.45044) (end 156.9593 78.4225) (width 1.2) (layer F.Cu) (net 8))
 (segment (start 177.1904 102.1842) (end 177.1904 98.5774) (width 1.4) (layer F.Cu) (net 8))
 (segment (start 175.5775 103.7971) (end 177.1904 102.1842) (width 1.4) (layer F.Cu) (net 8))
 (segment (start 166.5926 103.7971) (end 175.5775 103.7971) (width 1.4) (layer F.Cu) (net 8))
 (segment (start 163.1061 110.0836) (end 163.1061 107.2836) (width 1.4) (layer F.Cu) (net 8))
 (segment (start 163.1061 107.2836) (end 166.5926 103.7971) (width 1.4) (layer F.Cu) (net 8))
 (segment (start 168.1061 110.0836) (end 168.1061 107.2836) (width 1.4) (layer F.Cu) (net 21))
 (segment (start 168.1061 107.2836) (end 168.7732 106.6165) (width 1.4) (layer F.Cu) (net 21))
 (segment (start 168.7732 106.6165) (end 178.8033 106.6165) (width 1.4) (layer F.Cu) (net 21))
 (segment (start 178.8033 106.6165) (end 179.8066 105.6132) (width 1.4) (layer F.Cu) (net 21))
 (segment (start 176.70572 92.60632) (end 176.46269 92.60632) (width 1.4) (layer F.Cu) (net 21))
 (segment (start 179.8066 105.6132) (end 179.8066 95.7072) (width 1.4) (layer F.Cu) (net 21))
 (segment (start 179.8066 95.7072) (end 176.70572 92.60632) (width 1.4) (layer F.Cu) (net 21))
 (segment (start 176.46269 92.60632) (end 176.46269 90.44432) (width 1.3) (layer F.Cu) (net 21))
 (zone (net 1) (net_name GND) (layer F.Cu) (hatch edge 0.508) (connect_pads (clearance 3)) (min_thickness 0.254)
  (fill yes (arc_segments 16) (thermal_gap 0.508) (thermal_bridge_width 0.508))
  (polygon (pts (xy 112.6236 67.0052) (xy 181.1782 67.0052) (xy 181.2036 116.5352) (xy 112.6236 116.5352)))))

